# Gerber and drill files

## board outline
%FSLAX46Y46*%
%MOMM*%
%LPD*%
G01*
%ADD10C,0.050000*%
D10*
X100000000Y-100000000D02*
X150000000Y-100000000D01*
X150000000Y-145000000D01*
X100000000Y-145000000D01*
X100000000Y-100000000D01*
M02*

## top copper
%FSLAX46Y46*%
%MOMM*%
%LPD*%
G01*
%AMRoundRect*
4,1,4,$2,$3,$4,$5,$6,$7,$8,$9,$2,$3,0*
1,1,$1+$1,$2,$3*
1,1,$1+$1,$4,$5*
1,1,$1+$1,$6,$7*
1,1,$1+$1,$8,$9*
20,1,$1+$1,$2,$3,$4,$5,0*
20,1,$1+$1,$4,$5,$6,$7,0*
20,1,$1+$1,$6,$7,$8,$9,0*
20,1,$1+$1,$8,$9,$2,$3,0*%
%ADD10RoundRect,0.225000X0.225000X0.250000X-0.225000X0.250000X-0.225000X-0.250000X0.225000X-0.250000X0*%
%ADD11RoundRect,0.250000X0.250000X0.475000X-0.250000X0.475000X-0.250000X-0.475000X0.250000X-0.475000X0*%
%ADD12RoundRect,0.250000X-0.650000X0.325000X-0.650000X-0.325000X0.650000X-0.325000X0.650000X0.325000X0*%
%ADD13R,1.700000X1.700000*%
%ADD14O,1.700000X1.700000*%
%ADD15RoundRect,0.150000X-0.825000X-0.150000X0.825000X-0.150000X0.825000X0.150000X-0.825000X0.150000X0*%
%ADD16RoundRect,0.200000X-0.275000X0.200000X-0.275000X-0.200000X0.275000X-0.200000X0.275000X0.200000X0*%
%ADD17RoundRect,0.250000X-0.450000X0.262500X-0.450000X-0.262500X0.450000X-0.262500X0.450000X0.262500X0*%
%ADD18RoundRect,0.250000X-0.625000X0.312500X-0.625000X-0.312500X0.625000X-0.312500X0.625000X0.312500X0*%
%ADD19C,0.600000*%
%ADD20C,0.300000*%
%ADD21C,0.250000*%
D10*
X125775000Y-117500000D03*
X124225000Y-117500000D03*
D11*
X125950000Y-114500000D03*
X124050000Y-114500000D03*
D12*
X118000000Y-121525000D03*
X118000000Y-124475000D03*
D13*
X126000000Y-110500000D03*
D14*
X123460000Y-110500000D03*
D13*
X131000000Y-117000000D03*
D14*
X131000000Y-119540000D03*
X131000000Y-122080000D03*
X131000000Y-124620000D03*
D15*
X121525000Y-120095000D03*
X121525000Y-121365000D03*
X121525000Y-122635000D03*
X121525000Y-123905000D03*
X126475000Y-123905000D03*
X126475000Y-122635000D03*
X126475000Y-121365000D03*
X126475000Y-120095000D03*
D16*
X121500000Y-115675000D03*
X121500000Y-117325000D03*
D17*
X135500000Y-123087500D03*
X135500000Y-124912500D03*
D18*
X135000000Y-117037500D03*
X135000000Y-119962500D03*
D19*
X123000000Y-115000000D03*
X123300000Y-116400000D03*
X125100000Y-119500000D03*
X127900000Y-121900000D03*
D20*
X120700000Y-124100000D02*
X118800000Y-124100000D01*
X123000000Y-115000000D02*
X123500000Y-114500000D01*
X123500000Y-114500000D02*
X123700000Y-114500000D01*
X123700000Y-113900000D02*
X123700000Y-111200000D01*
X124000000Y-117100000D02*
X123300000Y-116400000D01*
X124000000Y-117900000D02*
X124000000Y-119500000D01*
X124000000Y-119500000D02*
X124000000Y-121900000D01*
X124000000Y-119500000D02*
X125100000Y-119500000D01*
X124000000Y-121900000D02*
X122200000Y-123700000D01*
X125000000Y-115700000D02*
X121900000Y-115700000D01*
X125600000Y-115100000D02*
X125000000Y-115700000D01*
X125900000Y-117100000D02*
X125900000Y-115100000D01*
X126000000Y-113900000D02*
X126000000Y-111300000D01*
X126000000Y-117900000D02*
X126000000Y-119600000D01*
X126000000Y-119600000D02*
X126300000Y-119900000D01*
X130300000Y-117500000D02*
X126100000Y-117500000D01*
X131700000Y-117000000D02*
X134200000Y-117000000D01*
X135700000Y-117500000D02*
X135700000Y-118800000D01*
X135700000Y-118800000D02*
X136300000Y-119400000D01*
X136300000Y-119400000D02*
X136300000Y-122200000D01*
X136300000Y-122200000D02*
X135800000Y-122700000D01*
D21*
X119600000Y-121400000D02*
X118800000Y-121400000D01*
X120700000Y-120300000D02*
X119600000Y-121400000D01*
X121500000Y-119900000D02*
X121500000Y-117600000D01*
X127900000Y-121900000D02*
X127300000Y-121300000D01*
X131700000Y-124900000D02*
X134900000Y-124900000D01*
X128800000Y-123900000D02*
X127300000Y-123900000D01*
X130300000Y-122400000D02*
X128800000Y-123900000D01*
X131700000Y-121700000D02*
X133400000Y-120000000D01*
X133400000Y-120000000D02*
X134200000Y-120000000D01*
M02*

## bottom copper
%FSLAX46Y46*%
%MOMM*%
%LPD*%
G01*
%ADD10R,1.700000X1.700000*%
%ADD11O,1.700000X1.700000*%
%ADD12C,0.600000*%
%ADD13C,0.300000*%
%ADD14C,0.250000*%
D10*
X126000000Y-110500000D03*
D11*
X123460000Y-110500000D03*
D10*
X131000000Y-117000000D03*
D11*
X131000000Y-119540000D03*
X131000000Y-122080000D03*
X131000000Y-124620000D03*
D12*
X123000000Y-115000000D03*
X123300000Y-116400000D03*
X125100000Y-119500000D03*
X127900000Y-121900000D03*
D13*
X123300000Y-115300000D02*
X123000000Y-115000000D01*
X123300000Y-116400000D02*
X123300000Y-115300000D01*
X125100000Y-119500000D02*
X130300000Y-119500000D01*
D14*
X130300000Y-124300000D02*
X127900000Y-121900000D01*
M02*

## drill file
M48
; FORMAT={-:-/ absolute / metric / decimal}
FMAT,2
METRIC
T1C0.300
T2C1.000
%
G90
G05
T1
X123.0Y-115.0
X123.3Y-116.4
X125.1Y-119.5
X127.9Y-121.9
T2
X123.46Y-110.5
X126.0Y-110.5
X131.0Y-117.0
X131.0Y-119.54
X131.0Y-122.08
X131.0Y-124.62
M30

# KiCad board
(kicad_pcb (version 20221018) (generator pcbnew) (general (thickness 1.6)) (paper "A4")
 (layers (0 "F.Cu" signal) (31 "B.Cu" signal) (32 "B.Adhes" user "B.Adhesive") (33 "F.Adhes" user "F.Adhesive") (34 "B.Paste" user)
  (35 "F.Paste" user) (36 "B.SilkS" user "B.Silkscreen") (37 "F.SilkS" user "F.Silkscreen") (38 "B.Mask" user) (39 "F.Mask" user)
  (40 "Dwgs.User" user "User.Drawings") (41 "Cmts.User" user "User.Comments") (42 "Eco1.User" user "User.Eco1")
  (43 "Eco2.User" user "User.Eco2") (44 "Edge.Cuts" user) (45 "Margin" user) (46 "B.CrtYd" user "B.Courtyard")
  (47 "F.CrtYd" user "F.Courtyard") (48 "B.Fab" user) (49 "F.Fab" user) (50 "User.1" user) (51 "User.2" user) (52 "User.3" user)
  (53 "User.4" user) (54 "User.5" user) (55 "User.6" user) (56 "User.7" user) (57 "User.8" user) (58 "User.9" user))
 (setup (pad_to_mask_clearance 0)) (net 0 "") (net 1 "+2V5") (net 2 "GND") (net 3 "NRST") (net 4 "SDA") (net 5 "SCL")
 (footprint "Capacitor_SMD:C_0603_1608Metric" (layer "F.Cu") (at 125 117.5 180)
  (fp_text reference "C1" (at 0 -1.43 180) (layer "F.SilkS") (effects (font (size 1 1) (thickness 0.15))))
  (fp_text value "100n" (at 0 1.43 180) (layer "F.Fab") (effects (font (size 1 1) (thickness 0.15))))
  (pad "1" smd roundrect (at -0.775 0 180) (size 0.9 0.95) (layers "F.Cu" "F.Paste" "F.Mask") (roundrect_rratio 0.25) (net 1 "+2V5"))
  (pad "2" smd roundrect (at 0.775 0 180) (size 0.9 0.95) (layers "F.Cu" "F.Paste" "F.Mask") (roundrect_rratio 0.25) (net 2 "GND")))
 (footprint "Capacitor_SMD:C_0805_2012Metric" (layer "F.Cu") (at 125 114.5 180)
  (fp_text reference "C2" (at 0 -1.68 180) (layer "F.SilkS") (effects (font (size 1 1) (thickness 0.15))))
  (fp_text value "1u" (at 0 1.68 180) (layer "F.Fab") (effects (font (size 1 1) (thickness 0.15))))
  (pad "1" smd roundrect (at -0.95 0 180) (size 1 1.45) (layers "F.Cu" "F.Paste" "F.Mask") (roundrect_rratio 0.25) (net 1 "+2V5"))
  (pad "2" smd roundrect (at 0.95 0 180) (size 1 1.45) (layers "F.Cu" "F.Paste" "F.Mask") (roundrect_rratio 0.25) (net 2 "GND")))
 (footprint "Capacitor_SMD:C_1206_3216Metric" (layer "F.Cu") (at 118 123 -90)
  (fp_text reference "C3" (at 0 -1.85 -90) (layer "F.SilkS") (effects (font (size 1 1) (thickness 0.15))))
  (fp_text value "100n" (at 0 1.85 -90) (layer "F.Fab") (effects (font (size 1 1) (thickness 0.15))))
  (pad "1" smd roundrect (at -1.475 0 270) (size 1.15 1.8) (layers "F.Cu" "F.Paste" "F.Mask") (roundrect_rratio 0.217391) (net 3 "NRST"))
  (pad "2" smd roundrect (at 1.475 0 270) (size 1.15 1.8) (layers "F.Cu" "F.Paste" "F.Mask") (roundrect_rratio 0.217391) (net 2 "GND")))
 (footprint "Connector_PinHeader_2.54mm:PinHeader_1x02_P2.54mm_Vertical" (layer "F.Cu") (at 126 110.5 -90)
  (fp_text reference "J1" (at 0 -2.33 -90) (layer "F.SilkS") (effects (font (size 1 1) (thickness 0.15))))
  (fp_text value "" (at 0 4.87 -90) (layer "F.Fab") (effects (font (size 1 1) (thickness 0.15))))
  (pad "1" thru_hole rect (at 0 0 270) (size 1.7 1.7) (drill 1) (layers "*.Cu" "*.Mask") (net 1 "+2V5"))
  (pad "2" thru_hole oval (at 0 2.54 270) (size 1.7 1.7) (drill 1) (layers "*.Cu" "*.Mask") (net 2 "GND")))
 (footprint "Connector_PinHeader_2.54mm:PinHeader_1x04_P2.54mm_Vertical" (layer "F.Cu") (at 131 117)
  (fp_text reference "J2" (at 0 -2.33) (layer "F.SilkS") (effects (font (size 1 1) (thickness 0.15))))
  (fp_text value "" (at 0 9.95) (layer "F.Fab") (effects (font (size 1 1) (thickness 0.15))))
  (pad "1" thru_hole rect (at 0 0) (size 1.7 1.7) (drill 1) (layers "*.Cu" "*.Mask") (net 1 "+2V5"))
  (pad "2" thru_hole oval (at 0 2.54) (size 1.7 1.7) (drill 1) (layers "*.Cu" "*.Mask") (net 2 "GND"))
  (pad "3" thru_hole oval (at 0 5.08) (size 1.7 1.7) (drill 1) (layers "*.Cu" "*.Mask") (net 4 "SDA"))
  (pad "4" thru_hole oval (at 0 7.62) (size 1.7 1.7) (drill 1) (layers "*.Cu" "*.Mask") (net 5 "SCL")))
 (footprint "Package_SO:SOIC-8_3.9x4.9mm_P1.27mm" (layer "F.Cu") (at 124 122)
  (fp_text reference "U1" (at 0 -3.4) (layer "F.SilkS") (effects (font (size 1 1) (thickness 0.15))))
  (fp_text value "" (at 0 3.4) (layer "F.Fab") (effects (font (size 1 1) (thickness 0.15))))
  (pad "1" smd roundrect (at -2.475 -1.905) (size 1.95 0.6) (layers "F.Cu" "F.Paste" "F.Mask") (roundrect_rratio 0.25) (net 3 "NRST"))
  (pad "2" smd roundrect (at -2.475 -0.635) (size 1.95 0.6) (layers "F.Cu" "F.Paste" "F.Mask") (roundrect_rratio 0.25))
  (pad "3" smd roundrect (at -2.475 0.635) (size 1.95 0.6) (layers "F.Cu" "F.Paste" "F.Mask") (roundrect_rratio 0.25))
  (pad "4" smd roundrect (at -2.475 1.905) (size 1.95 0.6) (layers "F.Cu" "F.Paste" "F.Mask") (roundrect_rratio 0.25) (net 2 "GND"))
  (pad "5" smd roundrect (at 2.475 1.905) (size 1.95 0.6) (layers "F.Cu" "F.Paste" "F.Mask") (roundrect_rratio 0.25) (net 4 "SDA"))
  (pad "6" smd roundrect (at 2.475 0.635) (size 1.95 0.6) (layers "F.Cu" "F.Paste" "F.Mask") (roundrect_rratio 0.25))
  (pad "7" smd roundrect (at 2.475 -0.635) (size 1.95 0.6) (layers "F.Cu" "F.Paste" "F.Mask") (roundrect_rratio 0.25) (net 5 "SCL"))
  (pad "8" smd roundrect (at 2.475 -1.905) (size 1.95 0.6) (layers "F.Cu" "F.Paste" "F.Mask") (roundrect_rratio 0.25) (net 1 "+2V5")))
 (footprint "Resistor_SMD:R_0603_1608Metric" (layer "F.Cu") (at 121.5 116.5 -90)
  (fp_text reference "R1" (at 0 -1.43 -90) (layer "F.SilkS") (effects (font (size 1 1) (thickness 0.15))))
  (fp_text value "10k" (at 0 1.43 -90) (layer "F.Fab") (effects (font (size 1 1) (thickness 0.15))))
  (pad "1" smd roundrect (at -0.825 0 270) (size 0.8 0.95) (layers "F.Cu" "F.Paste" "F.Mask") (roundrect_rratio 0.25) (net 1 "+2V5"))
  (pad "2" smd roundrect (at 0.825 0 270) (size 0.8 0.95) (layers "F.Cu" "F.Paste" "F.Mask") (roundrect_rratio 0.25) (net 3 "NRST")))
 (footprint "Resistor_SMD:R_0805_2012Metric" (layer "F.Cu") (at 135.5 124 -90)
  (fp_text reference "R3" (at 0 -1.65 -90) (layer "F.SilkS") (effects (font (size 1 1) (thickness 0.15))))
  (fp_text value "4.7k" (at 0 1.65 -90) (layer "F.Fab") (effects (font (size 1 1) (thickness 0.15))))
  (pad "1" smd roundrect (at -0.9125 0 270) (size 1.025 1.4) (layers "F.Cu" "F.Paste" "F.Mask") (roundrect_rratio 0.243902) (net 1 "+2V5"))
  (pad "2" smd roundrect (at 0.9125 0 270) (size 1.025 1.4) (layers "F.Cu" "F.Paste" "F.Mask") (roundrect_rratio 0.243902) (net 5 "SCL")))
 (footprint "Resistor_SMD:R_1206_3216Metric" (layer "F.Cu") (at 135 118.5 -90)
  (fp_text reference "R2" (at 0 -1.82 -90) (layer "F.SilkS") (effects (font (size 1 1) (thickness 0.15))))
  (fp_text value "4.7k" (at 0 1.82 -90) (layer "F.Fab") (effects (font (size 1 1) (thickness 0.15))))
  (pad "1" smd roundrect (at -1.4625 0 270) (size 1.125 1.75) (layers "F.Cu" "F.Paste" "F.Mask") (roundrect_rratio 0.222222) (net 1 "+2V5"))
  (pad "2" smd roundrect (at 1.4625 0 270) (size 1.125 1.75) (layers "F.Cu" "F.Paste" "F.Mask") (roundrect_rratio 0.222222) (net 4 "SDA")))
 (gr_rect (start 100 100) (end 150 145) (stroke (width 0.05) (type default)) (fill none) (layer "Edge.Cuts"))
 (segment (start 120.7 124.1) (end 118.8 124.1) (width 0.3) (layer "F.Cu") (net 2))
 (segment (start 123 115) (end 123.5 114.5) (width 0.3) (layer "F.Cu") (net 2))
 (segment (start 123.5 114.5) (end 123.7 114.5) (width 0.3) (layer "F.Cu") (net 2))
 (segment (start 123.7 113.9) (end 123.7 111.2) (width 0.3) (layer "F.Cu") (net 2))
 (segment (start 124 117.1) (end 123.3 116.4) (width 0.3) (layer "F.Cu") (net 2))
 (segment (start 124 117.9) (end 124 119.5) (width 0.3) (layer "F.Cu") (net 2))
 (segment (start 124 119.5) (end 124 121.9) (width 0.3) (layer "F.Cu") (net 2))
 (segment (start 124 119.5) (end 125.1 119.5) (width 0.3) (layer "F.Cu") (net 2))
 (segment (start 124 121.9) (end 122.2 123.7) (width 0.3) (layer "F.Cu") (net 2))
 (segment (start 125 115.7) (end 121.9 115.7) (width 0.3) (layer "F.Cu") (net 1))
 (segment (start 125.6 115.1) (end 125 115.7) (width 0.3) (layer "F.Cu") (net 1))
 (segment (start 125.9 117.1) (end 125.9 115.1) (width 0.3) (layer "F.Cu") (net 1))
 (segment (start 126 113.9) (end 126 111.3) (width 0.3) (layer "F.Cu") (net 1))
 (segment (start 126 117.9) (end 126 119.6) (width 0.3) (layer "F.Cu") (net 1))
 (segment (start 126 119.6) (end 126.3 119.9) (width 0.3) (layer "F.Cu") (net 1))
 (segment (start 130.3 117.5) (end 126.1 117.5) (width 0.3) (layer "F.Cu") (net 1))
 (segment (start 131.7 117) (end 134.2 117) (width 0.3) (layer "F.Cu") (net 1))
 (segment (start 135.7 117.5) (end 135.7 118.8) (width 0.3) (layer "F.Cu") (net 1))
 (segment (start 135.7 118.8) (end 136.3 119.4) (width 0.3) (layer "F.Cu") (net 1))
 (segment (start 136.3 119.4) (end 136.3 122.2) (width 0.3) (layer "F.Cu") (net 1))
 (segment (start 136.3 122.2) (end 135.8 122.7) (width 0.3) (layer "F.Cu") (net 1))
 (via (at 123 115) (size 0.6) (drill 0.3) (layers "F.Cu" "B.Cu") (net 2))
 (via (at 123.3 116.4) (size 0.6) (drill 0.3) (layers "F.Cu" "B.Cu") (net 2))
 (via (at 125.1 119.5) (size 0.6) (drill 0.3) (layers "F.Cu" "B.Cu") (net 2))
 (segment (start 119.6 121.4) (end 118.8 121.4) (width 0.25) (layer "F.Cu") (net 3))
 (segment (start 120.7 120.3) (end 119.6 121.4) (width 0.25) (layer "F.Cu") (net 3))
 (segment (start 121.5 119.9) (end 121.5 117.6) (width 0.25) (layer "F.Cu") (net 3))
 (segment (start 123.3 115.3) (end 123 115) (width 0.3) (layer "B.Cu") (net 2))
 (segment (start 123.3 116.4) (end 123.3 115.3) (width 0.3) (layer "B.Cu") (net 2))
 (segment (start 125.1 119.5) (end 130.3 119.5) (width 0.3) (layer "B.Cu") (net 2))
 (segment (start 127.9 121.9) (end 127.3 121.3) (width 0.25) (layer "F.Cu") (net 5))
 (segment (start 131.7 124.9) (end 134.9 124.9) (width 0.25) (layer "F.Cu") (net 5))
 (via (at 127.9 121.9) (size 0.6) (drill 0.3) (layers "F.Cu" "B.Cu") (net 5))
 (segment (start 128.8 123.9) (end 127.3 123.9) (width 0.25) (layer "F.Cu") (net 4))
 (segment (start 130.3 122.4) (end 128.8 123.9) (width 0.25) (layer "F.Cu") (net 4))
 (segment (start 130.3 124.3) (end 127.9 121.9) (width 0.25) (layer "B.Cu") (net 5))
 (segment (start 131.7 121.7) (end 133.4 120) (width 0.25) (layer "F.Cu") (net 4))
 (segment (start 133.4 120) (end 134.2 120) (width 0.25) (layer "F.Cu") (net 4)))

